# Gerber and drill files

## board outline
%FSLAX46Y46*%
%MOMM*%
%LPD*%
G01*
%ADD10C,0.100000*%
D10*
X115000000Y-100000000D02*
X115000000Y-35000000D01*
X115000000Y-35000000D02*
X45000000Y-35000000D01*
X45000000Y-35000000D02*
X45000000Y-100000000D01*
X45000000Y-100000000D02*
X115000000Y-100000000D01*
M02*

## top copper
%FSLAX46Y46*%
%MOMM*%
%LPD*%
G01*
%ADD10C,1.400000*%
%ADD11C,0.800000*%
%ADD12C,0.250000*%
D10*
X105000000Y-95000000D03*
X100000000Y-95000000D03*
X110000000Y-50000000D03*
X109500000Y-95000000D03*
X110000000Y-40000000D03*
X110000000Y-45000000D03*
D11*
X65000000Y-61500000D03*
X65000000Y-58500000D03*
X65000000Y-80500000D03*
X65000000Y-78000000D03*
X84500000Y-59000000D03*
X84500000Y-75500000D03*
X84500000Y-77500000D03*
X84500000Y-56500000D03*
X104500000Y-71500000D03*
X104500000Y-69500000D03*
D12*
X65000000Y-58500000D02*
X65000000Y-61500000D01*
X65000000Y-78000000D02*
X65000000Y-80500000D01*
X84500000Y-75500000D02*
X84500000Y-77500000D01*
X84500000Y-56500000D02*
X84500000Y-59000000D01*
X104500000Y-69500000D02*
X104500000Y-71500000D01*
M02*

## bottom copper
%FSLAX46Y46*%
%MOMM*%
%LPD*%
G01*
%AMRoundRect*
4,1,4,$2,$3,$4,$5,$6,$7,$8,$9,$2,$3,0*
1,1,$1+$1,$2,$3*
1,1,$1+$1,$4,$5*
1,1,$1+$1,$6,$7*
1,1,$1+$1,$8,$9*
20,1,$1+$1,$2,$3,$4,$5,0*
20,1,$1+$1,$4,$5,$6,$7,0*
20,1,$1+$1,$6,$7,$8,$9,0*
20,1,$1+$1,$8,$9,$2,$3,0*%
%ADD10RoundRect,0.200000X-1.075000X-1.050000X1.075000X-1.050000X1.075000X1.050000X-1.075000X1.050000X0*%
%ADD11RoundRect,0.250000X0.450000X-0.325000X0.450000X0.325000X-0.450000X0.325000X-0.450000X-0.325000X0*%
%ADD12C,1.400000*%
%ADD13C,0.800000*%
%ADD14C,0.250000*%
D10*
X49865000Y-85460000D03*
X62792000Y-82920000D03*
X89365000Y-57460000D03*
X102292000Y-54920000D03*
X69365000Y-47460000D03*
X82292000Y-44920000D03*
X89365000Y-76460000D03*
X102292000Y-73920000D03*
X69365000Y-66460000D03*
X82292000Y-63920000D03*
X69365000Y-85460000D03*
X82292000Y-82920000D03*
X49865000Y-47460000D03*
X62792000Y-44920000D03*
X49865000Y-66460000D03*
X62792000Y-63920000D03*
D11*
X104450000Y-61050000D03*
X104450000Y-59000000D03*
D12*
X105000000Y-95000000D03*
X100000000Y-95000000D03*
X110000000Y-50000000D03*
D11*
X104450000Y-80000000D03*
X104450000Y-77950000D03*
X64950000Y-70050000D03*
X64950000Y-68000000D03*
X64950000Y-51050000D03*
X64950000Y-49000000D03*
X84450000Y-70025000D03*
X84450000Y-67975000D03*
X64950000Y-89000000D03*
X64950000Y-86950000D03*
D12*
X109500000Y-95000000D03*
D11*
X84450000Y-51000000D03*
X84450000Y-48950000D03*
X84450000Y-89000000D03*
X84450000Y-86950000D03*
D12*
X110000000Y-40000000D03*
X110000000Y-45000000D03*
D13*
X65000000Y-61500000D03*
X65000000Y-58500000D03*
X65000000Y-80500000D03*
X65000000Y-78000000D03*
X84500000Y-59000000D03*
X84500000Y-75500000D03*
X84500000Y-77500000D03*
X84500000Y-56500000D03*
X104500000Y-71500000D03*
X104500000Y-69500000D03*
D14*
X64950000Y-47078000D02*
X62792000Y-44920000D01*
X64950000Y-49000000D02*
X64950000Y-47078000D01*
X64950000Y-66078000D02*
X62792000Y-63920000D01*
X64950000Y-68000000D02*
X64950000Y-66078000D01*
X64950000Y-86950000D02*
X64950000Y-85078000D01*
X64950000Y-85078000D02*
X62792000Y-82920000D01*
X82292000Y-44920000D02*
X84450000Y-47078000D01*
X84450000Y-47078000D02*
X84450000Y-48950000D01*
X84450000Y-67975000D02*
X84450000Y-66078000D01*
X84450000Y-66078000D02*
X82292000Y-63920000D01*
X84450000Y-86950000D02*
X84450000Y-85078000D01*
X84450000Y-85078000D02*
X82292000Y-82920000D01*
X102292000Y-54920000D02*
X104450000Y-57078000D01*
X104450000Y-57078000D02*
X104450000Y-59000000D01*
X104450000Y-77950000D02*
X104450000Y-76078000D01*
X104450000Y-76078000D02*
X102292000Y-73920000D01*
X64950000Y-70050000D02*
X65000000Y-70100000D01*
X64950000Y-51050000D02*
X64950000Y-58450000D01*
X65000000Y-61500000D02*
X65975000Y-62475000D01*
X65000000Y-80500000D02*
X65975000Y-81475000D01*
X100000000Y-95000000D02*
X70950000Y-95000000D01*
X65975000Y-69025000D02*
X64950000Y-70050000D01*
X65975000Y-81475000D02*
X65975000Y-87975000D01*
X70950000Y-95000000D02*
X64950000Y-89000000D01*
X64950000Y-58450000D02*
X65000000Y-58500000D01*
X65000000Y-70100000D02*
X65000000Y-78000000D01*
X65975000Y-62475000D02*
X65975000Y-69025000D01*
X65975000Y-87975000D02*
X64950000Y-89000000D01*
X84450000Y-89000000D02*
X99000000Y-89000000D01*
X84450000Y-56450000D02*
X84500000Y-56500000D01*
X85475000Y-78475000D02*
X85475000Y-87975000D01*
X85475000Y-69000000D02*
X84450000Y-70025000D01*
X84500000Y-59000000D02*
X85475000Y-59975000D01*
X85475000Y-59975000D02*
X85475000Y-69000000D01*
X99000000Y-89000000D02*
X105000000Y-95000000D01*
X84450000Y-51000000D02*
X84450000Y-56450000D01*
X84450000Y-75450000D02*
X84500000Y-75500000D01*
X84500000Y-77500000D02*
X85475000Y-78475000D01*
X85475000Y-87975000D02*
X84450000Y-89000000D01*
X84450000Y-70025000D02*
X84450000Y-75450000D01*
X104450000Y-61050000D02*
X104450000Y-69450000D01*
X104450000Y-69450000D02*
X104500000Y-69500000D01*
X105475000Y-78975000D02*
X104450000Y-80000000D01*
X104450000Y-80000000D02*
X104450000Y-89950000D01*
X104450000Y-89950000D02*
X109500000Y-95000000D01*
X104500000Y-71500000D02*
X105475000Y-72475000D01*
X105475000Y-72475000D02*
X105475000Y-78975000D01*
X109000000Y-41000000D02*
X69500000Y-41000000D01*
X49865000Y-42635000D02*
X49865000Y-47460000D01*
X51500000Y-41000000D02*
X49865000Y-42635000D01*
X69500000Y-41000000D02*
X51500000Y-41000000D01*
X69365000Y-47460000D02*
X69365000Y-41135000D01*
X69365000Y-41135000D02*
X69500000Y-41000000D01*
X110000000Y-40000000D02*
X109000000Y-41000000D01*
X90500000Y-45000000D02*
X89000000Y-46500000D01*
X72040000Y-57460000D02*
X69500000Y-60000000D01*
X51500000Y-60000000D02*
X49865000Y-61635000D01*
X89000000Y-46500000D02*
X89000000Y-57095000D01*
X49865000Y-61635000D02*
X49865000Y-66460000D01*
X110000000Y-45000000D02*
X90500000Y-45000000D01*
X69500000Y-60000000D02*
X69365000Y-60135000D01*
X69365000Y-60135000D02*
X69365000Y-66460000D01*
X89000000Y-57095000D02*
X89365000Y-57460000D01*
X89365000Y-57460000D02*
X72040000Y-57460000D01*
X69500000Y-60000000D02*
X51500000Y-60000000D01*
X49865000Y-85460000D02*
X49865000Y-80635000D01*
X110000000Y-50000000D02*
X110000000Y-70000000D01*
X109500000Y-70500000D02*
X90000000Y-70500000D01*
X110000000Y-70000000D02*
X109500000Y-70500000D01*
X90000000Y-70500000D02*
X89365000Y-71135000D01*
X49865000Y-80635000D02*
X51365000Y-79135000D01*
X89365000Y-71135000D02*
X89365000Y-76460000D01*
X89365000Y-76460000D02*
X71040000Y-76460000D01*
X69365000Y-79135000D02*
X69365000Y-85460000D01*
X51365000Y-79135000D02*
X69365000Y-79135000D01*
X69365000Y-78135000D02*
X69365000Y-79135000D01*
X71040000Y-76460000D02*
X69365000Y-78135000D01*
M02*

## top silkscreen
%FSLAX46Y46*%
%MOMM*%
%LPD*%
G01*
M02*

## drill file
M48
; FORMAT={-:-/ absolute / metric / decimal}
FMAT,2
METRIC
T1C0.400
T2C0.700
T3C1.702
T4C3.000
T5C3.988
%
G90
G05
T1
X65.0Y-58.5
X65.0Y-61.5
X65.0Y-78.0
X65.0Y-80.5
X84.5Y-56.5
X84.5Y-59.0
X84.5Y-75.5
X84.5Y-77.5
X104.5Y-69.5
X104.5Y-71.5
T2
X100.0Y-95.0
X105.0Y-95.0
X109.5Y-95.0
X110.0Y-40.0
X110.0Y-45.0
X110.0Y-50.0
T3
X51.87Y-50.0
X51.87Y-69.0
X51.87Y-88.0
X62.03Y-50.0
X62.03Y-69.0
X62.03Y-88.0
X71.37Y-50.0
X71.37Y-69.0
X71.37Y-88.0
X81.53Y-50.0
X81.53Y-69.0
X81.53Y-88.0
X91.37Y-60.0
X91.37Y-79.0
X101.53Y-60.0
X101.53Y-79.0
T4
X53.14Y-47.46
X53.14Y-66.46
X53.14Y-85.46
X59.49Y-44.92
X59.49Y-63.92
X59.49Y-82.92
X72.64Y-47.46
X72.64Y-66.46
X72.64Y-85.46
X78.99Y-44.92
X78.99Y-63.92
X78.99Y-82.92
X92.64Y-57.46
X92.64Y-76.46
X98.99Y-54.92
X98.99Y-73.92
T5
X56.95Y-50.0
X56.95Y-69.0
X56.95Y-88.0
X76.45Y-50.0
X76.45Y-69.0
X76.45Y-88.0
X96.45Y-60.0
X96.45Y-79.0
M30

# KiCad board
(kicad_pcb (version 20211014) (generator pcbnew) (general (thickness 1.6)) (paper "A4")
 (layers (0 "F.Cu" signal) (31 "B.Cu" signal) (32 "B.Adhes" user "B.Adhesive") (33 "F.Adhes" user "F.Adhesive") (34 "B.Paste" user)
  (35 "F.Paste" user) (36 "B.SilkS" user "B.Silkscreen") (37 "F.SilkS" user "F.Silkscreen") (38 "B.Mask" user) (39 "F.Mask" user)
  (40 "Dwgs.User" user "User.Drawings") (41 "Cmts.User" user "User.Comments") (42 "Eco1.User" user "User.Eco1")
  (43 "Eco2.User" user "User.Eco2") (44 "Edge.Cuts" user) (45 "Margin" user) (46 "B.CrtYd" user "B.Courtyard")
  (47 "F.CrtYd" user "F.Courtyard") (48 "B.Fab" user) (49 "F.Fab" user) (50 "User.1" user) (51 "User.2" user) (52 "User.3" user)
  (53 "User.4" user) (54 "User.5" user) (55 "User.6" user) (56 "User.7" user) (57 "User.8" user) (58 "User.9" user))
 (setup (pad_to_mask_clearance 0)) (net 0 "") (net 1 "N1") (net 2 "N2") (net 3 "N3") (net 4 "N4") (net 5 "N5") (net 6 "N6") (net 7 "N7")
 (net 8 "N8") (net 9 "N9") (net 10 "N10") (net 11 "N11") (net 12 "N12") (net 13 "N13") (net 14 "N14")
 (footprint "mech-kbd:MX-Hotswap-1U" (layer "F.Cu") (at 56.95 88)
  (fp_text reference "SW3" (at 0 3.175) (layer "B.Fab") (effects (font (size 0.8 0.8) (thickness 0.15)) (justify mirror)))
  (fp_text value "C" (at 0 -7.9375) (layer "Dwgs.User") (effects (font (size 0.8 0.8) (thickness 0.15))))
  (pad "" np_thru_hole circle (at 2.54 -5.08) (size 3 3) (drill 3) (layers F&B.Cu *.Mask))
  (pad "" np_thru_hole circle (at -3.81 -2.54) (size 3 3) (drill 3) (layers F&B.Cu *.Mask))
  (pad "" np_thru_hole circle (at 0 0) (size 3.9878 3.9878) (drill 3.9878) (layers F&B.Cu *.Mask))
  (pad "" np_thru_hole circle (at -5.08 0 48.099) (size 1.7018 1.7018) (drill 1.7018) (layers F&B.Cu *.Mask))
  (pad "" np_thru_hole circle (at 5.08 0 48.099) (size 1.7018 1.7018) (drill 1.7018) (layers F&B.Cu *.Mask))
  (pad "1" smd roundrect (at -7.085 -2.54) (size 2.55 2.5) (layers "B.Cu" "B.Paste" "B.Mask") (roundrect_rratio 0.08) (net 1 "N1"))
  (pad "2" smd roundrect (at 5.842 -5.08) (size 2.55 2.5) (layers "B.Cu" "B.Paste" "B.Mask") (roundrect_rratio 0.08) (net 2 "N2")))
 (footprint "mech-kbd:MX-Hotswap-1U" (layer "F.Cu") (at 96.45 60)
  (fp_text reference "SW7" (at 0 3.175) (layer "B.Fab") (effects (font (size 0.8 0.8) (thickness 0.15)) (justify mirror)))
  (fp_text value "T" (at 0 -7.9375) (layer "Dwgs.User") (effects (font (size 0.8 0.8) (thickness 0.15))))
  (pad "" np_thru_hole circle (at 5.08 0 48.099) (size 1.7018 1.7018) (drill 1.7018) (layers F&B.Cu *.Mask))
  (pad "" np_thru_hole circle (at 0 0) (size 3.9878 3.9878) (drill 3.9878) (layers F&B.Cu *.Mask))
  (pad "" np_thru_hole circle (at -3.81 -2.54) (size 3 3) (drill 3) (layers F&B.Cu *.Mask))
  (pad "" np_thru_hole circle (at 2.54 -5.08) (size 3 3) (drill 3) (layers F&B.Cu *.Mask))
  (pad "" np_thru_hole circle (at -5.08 0 48.099) (size 1.7018 1.7018) (drill 1.7018) (layers F&B.Cu *.Mask))
  (pad "1" smd roundrect (at -7.085 -2.54) (size 2.55 2.5) (layers "B.Cu" "B.Paste" "B.Mask") (roundrect_rratio 0.08) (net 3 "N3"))
  (pad "2" smd roundrect (at 5.842 -5.08) (size 2.55 2.5) (layers "B.Cu" "B.Paste" "B.Mask") (roundrect_rratio 0.08) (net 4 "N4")))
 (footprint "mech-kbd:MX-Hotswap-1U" (layer "F.Cu") (at 76.45 50)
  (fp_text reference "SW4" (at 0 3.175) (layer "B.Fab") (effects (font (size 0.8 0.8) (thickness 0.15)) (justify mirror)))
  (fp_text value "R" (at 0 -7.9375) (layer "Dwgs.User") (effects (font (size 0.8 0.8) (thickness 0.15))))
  (pad "" np_thru_hole circle (at 2.54 -5.08) (size 3 3) (drill 3) (layers F&B.Cu *.Mask))
  (pad "" np_thru_hole circle (at -3.81 -2.54) (size 3 3) (drill 3) (layers F&B.Cu *.Mask))
  (pad "" np_thru_hole circle (at 5.08 0 48.099) (size 1.7018 1.7018) (drill 1.7018) (layers F&B.Cu *.Mask))
  (pad "" np_thru_hole circle (at 0 0) (size 3.9878 3.9878) (drill 3.9878) (layers F&B.Cu *.Mask))
  (pad "" np_thru_hole circle (at -5.08 0 48.099) (size 1.7018 1.7018) (drill 1.7018) (layers F&B.Cu *.Mask))
  (pad "1" smd roundrect (at -7.085 -2.54) (size 2.55 2.5) (layers "B.Cu" "B.Paste" "B.Mask") (roundrect_rratio 0.08) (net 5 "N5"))
  (pad "2" smd roundrect (at 5.842 -5.08) (size 2.55 2.5) (layers "B.Cu" "B.Paste" "B.Mask") (roundrect_rratio 0.08) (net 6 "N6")))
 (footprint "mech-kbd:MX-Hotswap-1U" (layer "F.Cu") (at 96.45 79)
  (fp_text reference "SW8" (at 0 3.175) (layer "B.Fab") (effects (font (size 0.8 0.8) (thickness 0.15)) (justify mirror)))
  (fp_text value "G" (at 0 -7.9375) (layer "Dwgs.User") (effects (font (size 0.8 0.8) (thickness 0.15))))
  (pad "" np_thru_hole circle (at 0 0) (size 3.9878 3.9878) (drill 3.9878) (layers F&B.Cu *.Mask))
  (pad "" np_thru_hole circle (at 2.54 -5.08) (size 3 3) (drill 3) (layers F&B.Cu *.Mask))
  (pad "" np_thru_hole circle (at -3.81 -2.54) (size 3 3) (drill 3) (layers F&B.Cu *.Mask))
  (pad "" np_thru_hole circle (at 5.08 0 48.099) (size 1.7018 1.7018) (drill 1.7018) (layers F&B.Cu *.Mask))
  (pad "" np_thru_hole circle (at -5.08 0 48.099) (size 1.7018 1.7018) (drill 1.7018) (layers F&B.Cu *.Mask))
  (pad "1" smd roundrect (at -7.085 -2.54) (size 2.55 2.5) (layers "B.Cu" "B.Paste" "B.Mask") (roundrect_rratio 0.08) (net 1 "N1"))
  (pad "2" smd roundrect (at 5.842 -5.08) (size 2.55 2.5) (layers "B.Cu" "B.Paste" "B.Mask") (roundrect_rratio 0.08) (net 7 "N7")))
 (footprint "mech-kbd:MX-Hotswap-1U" (layer "F.Cu") (at 76.45 69)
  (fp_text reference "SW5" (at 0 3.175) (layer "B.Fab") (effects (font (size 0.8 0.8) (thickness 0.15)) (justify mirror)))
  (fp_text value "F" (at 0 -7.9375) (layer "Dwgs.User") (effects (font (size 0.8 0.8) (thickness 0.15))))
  (pad "" np_thru_hole circle (at 5.08 0 48.099) (size 1.7018 1.7018) (drill 1.7018) (layers F&B.Cu *.Mask))
  (pad "" np_thru_hole circle (at 2.54 -5.08) (size 3 3) (drill 3) (layers F&B.Cu *.Mask))
  (pad "" np_thru_hole circle (at -3.81 -2.54) (size 3 3) (drill 3) (layers F&B.Cu *.Mask))
  (pad "" np_thru_hole circle (at -5.08 0 48.099) (size 1.7018 1.7018) (drill 1.7018) (layers F&B.Cu *.Mask))
  (pad "" np_thru_hole circle (at 0 0) (size 3.9878 3.9878) (drill 3.9878) (layers F&B.Cu *.Mask))
  (pad "1" smd roundrect (at -7.085 -2.54) (size 2.55 2.5) (layers "B.Cu" "B.Paste" "B.Mask") (roundrect_rratio 0.08) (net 3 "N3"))
  (pad "2" smd roundrect (at 5.842 -5.08) (size 2.55 2.5) (layers "B.Cu" "B.Paste" "B.Mask") (roundrect_rratio 0.08) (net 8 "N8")))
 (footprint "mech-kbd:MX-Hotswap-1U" (layer "F.Cu") (at 76.45 88)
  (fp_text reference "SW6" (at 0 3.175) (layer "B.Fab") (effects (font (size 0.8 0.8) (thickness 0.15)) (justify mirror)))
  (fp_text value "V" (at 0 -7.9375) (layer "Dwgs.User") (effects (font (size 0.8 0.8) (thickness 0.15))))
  (pad "" np_thru_hole circle (at -3.81 -2.54) (size 3 3) (drill 3) (layers F&B.Cu *.Mask))
  (pad "" np_thru_hole circle (at 0 0) (size 3.9878 3.9878) (drill 3.9878) (layers F&B.Cu *.Mask))
  (pad "" np_thru_hole circle (at 5.08 0 48.099) (size 1.7018 1.7018) (drill 1.7018) (layers F&B.Cu *.Mask))
  (pad "" np_thru_hole circle (at -5.08 0 48.099) (size 1.7018 1.7018) (drill 1.7018) (layers F&B.Cu *.Mask))
  (pad "" np_thru_hole circle (at 2.54 -5.08) (size 3 3) (drill 3) (layers F&B.Cu *.Mask))
  (pad "1" smd roundrect (at -7.085 -2.54) (size 2.55 2.5) (layers "B.Cu" "B.Paste" "B.Mask") (roundrect_rratio 0.08) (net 1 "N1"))
  (pad "2" smd roundrect (at 5.842 -5.08) (size 2.55 2.5) (layers "B.Cu" "B.Paste" "B.Mask") (roundrect_rratio 0.08) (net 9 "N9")))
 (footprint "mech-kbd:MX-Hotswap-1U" (layer "F.Cu") (at 56.95 50)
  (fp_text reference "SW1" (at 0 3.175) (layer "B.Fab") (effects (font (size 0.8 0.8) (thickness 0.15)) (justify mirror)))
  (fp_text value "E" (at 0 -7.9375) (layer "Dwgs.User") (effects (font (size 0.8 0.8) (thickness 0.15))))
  (pad "" np_thru_hole circle (at 5.08 0 48.099) (size 1.7018 1.7018) (drill 1.7018) (layers F&B.Cu *.Mask))
  (pad "" np_thru_hole circle (at 2.54 -5.08) (size 3 3) (drill 3) (layers F&B.Cu *.Mask))
  (pad "" np_thru_hole circle (at -5.08 0 48.099) (size 1.7018 1.7018) (drill 1.7018) (layers F&B.Cu *.Mask))
  (pad "" np_thru_hole circle (at 0 0) (size 3.9878 3.9878) (drill 3.9878) (layers F&B.Cu *.Mask))
  (pad "" np_thru_hole circle (at -3.81 -2.54) (size 3 3) (drill 3) (layers F&B.Cu *.Mask))
  (pad "1" smd roundrect (at -7.085 -2.54) (size 2.55 2.5) (layers "B.Cu" "B.Paste" "B.Mask") (roundrect_rratio 0.08) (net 5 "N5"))
  (pad "2" smd roundrect (at 5.842 -5.08) (size 2.55 2.5) (layers "B.Cu" "B.Paste" "B.Mask") (roundrect_rratio 0.08) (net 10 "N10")))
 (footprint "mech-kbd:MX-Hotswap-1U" (layer "F.Cu") (at 56.95 69)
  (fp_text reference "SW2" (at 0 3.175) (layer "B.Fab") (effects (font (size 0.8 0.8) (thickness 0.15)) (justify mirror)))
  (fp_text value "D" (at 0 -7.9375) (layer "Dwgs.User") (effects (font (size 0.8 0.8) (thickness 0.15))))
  (pad "" np_thru_hole circle (at 0 0) (size 3.9878 3.9878) (drill 3.9878) (layers F&B.Cu *.Mask))
  (pad "" np_thru_hole circle (at -3.81 -2.54) (size 3 3) (drill 3) (layers F&B.Cu *.Mask))
  (pad "" np_thru_hole circle (at -5.08 0 48.099) (size 1.7018 1.7018) (drill 1.7018) (layers F&B.Cu *.Mask))
  (pad "" np_thru_hole circle (at 5.08 0 48.099) (size 1.7018 1.7018) (drill 1.7018) (layers F&B.Cu *.Mask))
  (pad "" np_thru_hole circle (at 2.54 -5.08) (size 3 3) (drill 3) (layers F&B.Cu *.Mask))
  (pad "1" smd roundrect (at -7.085 -2.54) (size 2.55 2.5) (layers "B.Cu" "B.Paste" "B.Mask") (roundrect_rratio 0.08) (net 3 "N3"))
  (pad "2" smd roundrect (at 5.842 -5.08) (size 2.55 2.5) (layers "B.Cu" "B.Paste" "B.Mask") (roundrect_rratio 0.08) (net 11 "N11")))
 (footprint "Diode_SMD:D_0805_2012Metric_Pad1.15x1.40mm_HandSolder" (layer "B.Cu") (at 104.45 60.025 90)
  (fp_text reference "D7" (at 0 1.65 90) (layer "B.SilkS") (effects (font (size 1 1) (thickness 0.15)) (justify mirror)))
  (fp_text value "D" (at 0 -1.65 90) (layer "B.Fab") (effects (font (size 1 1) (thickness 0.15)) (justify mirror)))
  (pad "1" smd roundrect (at -1.025 0 90) (size 1.15 1.4) (layers "B.Cu" "B.Paste" "B.Mask") (roundrect_rratio 0.2173913043) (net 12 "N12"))
  (pad "2" smd roundrect (at 1.025 0 90) (size 1.15 1.4) (layers "B.Cu" "B.Paste" "B.Mask") (roundrect_rratio 0.2173913043) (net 4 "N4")))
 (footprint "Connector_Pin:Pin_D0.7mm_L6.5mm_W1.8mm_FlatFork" (layer "B.Cu") (at 105 95 180)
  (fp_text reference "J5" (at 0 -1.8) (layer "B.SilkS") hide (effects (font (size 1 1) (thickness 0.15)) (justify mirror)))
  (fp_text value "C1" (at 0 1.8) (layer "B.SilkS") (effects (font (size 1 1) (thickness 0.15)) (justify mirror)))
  (pad "1" thru_hole circle (at 0 0 180) (size 1.4 1.4) (drill 0.7) (layers *.Cu *.Mask) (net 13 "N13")))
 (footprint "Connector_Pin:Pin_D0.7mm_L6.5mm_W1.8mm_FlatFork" (layer "B.Cu") (at 100 95 180)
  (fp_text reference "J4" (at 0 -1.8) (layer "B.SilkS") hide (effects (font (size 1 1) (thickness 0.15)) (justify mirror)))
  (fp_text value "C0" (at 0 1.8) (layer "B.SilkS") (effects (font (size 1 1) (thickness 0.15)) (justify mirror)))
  (pad "1" thru_hole circle (at 0 0 180) (size 1.4 1.4) (drill 0.7) (layers *.Cu *.Mask) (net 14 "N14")))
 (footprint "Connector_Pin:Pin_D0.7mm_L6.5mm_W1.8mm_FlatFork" (layer "B.Cu") (at 110 50 180)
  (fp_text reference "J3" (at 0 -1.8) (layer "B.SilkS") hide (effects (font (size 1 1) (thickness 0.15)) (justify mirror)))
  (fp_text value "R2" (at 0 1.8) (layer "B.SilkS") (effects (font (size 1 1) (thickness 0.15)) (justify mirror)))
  (pad "1" thru_hole circle (at 0 0 180) (size 1.4 1.4) (drill 0.7) (layers *.Cu *.Mask) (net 1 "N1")))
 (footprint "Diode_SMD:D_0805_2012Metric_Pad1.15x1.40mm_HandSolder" (layer "B.Cu") (at 104.45 78.975 90)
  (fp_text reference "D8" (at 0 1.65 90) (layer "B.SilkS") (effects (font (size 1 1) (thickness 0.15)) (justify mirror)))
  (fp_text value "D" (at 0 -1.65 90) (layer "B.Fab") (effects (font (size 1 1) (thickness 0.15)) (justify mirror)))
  (pad "1" smd roundrect (at -1.025 0 90) (size 1.15 1.4) (layers "B.Cu" "B.Paste" "B.Mask") (roundrect_rratio 0.2173913043) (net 12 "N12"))
  (pad "2" smd roundrect (at 1.025 0 90) (size 1.15 1.4) (layers "B.Cu" "B.Paste" "B.Mask") (roundrect_rratio 0.2173913043) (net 7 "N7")))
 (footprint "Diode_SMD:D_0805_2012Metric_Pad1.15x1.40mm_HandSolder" (layer "B.Cu") (at 64.95 69.025 90)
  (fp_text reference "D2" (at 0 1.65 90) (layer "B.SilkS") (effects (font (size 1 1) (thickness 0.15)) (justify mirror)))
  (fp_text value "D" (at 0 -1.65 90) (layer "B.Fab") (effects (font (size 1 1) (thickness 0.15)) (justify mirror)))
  (pad "1" smd roundrect (at -1.025 0 90) (size 1.15 1.4) (layers "B.Cu" "B.Paste" "B.Mask") (roundrect_rratio 0.2173913043) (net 14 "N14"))
  (pad "2" smd roundrect (at 1.025 0 90) (size 1.15 1.4) (layers "B.Cu" "B.Paste" "B.Mask") (roundrect_rratio 0.2173913043) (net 11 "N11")))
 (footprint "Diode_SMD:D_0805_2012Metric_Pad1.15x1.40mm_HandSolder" (layer "B.Cu") (at 64.95 50.025 90)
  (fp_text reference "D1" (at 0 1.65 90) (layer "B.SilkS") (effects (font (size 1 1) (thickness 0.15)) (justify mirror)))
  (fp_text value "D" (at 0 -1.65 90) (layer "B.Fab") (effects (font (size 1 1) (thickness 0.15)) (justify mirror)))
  (pad "1" smd roundrect (at -1.025 0 90) (size 1.15 1.4) (layers "B.Cu" "B.Paste" "B.Mask") (roundrect_rratio 0.2173913043) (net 14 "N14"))
  (pad "2" smd roundrect (at 1.025 0 90) (size 1.15 1.4) (layers "B.Cu" "B.Paste" "B.Mask") (roundrect_rratio 0.2173913043) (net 10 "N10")))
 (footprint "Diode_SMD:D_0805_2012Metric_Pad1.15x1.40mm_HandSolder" (layer "B.Cu") (at 84.45 69 90)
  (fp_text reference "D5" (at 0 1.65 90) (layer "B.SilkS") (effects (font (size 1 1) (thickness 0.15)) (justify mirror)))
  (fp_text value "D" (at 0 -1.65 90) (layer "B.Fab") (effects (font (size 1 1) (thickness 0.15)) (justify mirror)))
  (pad "1" smd roundrect (at -1.025 0 90) (size 1.15 1.4) (layers "B.Cu" "B.Paste" "B.Mask") (roundrect_rratio 0.2173913043) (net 13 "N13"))
  (pad "2" smd roundrect (at 1.025 0 90) (size 1.15 1.4) (layers "B.Cu" "B.Paste" "B.Mask") (roundrect_rratio 0.2173913043) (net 8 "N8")))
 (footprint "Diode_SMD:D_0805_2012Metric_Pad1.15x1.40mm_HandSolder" (layer "B.Cu") (at 64.95 87.975 90)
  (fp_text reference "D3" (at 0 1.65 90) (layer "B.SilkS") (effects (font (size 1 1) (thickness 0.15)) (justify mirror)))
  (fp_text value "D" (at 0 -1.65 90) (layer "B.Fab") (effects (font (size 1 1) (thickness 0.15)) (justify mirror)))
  (pad "1" smd roundrect (at -1.025 0 90) (size 1.15 1.4) (layers "B.Cu" "B.Paste" "B.Mask") (roundrect_rratio 0.2173913043) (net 14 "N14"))
  (pad "2" smd roundrect (at 1.025 0 90) (size 1.15 1.4) (layers "B.Cu" "B.Paste" "B.Mask") (roundrect_rratio 0.2173913043) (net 2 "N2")))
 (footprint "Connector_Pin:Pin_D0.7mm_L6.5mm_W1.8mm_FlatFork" (layer "B.Cu") (at 109.5 95 180)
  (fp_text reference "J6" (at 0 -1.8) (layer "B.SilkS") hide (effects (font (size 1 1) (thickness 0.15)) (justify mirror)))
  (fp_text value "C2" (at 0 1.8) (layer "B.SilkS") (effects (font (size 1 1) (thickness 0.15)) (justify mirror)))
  (pad "1" thru_hole circle (at 0 0 180) (size 1.4 1.4) (drill 0.7) (layers *.Cu *.Mask) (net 12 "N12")))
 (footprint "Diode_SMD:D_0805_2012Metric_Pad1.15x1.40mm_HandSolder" (layer "B.Cu") (at 84.45 49.975 90)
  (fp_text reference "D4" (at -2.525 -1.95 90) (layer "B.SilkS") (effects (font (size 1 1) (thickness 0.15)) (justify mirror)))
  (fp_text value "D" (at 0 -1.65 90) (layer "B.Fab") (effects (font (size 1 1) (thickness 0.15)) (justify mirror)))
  (pad "1" smd roundrect (at -1.025 0 90) (size 1.15 1.4) (layers "B.Cu" "B.Paste" "B.Mask") (roundrect_rratio 0.2173913043) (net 13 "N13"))
  (pad "2" smd roundrect (at 1.025 0 90) (size 1.15 1.4) (layers "B.Cu" "B.Paste" "B.Mask") (roundrect_rratio 0.2173913043) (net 6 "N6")))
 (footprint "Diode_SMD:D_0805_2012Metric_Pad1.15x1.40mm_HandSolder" (layer "B.Cu") (at 84.45 87.975 90)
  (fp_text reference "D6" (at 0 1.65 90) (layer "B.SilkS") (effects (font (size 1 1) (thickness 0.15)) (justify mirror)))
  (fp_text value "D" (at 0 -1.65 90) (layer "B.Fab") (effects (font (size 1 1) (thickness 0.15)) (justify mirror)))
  (pad "1" smd roundrect (at -1.025 0 90) (size 1.15 1.4) (layers "B.Cu" "B.Paste" "B.Mask") (roundrect_rratio 0.2173913043) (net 13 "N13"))
  (pad "2" smd roundrect (at 1.025 0 90) (size 1.15 1.4) (layers "B.Cu" "B.Paste" "B.Mask") (roundrect_rratio 0.2173913043) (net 9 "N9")))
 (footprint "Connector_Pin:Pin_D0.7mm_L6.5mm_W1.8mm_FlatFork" (layer "B.Cu") (at 110 40 180)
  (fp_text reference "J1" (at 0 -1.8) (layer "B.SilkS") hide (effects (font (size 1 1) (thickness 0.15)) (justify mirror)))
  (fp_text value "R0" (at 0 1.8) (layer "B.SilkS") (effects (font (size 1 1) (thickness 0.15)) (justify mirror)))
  (pad "1" thru_hole circle (at 0 0 180) (size 1.4 1.4) (drill 0.7) (layers *.Cu *.Mask) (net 5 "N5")))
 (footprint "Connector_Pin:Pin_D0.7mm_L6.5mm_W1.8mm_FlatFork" (layer "B.Cu") (at 110 45 180)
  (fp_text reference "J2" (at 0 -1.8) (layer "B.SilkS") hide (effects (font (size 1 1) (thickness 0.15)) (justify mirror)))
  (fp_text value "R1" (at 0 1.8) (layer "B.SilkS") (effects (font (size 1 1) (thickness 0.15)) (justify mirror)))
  (pad "1" thru_hole circle (at 0 0 180) (size 1.4 1.4) (drill 0.7) (layers *.Cu *.Mask) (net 3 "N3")))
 (gr_line (start 115 100) (end 115 35) (layer "Edge.Cuts") (width 0.1))
 (gr_line (start 115 35) (end 45 35) (layer "Edge.Cuts") (width 0.1))
 (gr_line (start 45 35) (end 45 100) (layer "Edge.Cuts") (width 0.1))
 (gr_line (start 45 100) (end 115 100) (layer "Edge.Cuts") (width 0.1))
 (segment (start 64.95 47.078) (end 62.792 44.92) (width 0.25) (layer "B.Cu") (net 10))
 (segment (start 64.95 49) (end 64.95 47.078) (width 0.25) (layer "B.Cu") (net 10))
 (segment (start 64.95 66.078) (end 62.792 63.92) (width 0.25) (layer "B.Cu") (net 11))
 (segment (start 64.95 68) (end 64.95 66.078) (width 0.25) (layer "B.Cu") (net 11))
 (segment (start 64.95 86.95) (end 64.95 85.078) (width 0.25) (layer "B.Cu") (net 2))
 (segment (start 64.95 85.078) (end 62.792 82.92) (width 0.25) (layer "B.Cu") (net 2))
 (segment (start 82.292 44.92) (end 84.45 47.078) (width 0.25) (layer "B.Cu") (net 6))
 (segment (start 84.45 47.078) (end 84.45 48.95) (width 0.25) (layer "B.Cu") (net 6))
 (segment (start 84.45 67.975) (end 84.45 66.078) (width 0.25) (layer "B.Cu") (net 8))
 (segment (start 84.45 66.078) (end 82.292 63.92) (width 0.25) (layer "B.Cu") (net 8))
 (segment (start 84.45 86.95) (end 84.45 85.078) (width 0.25) (layer "B.Cu") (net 9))
 (segment (start 84.45 85.078) (end 82.292 82.92) (width 0.25) (layer "B.Cu") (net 9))
 (segment (start 102.292 54.92) (end 104.45 57.078) (width 0.25) (layer "B.Cu") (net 4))
 (segment (start 104.45 57.078) (end 104.45 59) (width 0.25) (layer "B.Cu") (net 4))
 (segment (start 104.45 77.95) (end 104.45 76.078) (width 0.25) (layer "B.Cu") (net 7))
 (segment (start 104.45 76.078) (end 102.292 73.92) (width 0.25) (layer "B.Cu") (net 7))
 (segment (start 65 58.5) (end 65 61.5) (width 0.25) (layer "F.Cu") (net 14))
 (segment (start 65 78) (end 65 80.5) (width 0.25) (layer "F.Cu") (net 14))
 (via (at 65 61.5) (size 0.8) (drill 0.4) (layers "F.Cu" "B.Cu") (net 14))
 (via (at 65 58.5) (size 0.8) (drill 0.4) (layers "F.Cu" "B.Cu") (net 14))
 (via (at 65 80.5) (size 0.8) (drill 0.4) (layers "F.Cu" "B.Cu") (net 14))
 (via (at 65 78) (size 0.8) (drill 0.4) (layers "F.Cu" "B.Cu") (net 14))
 (segment (start 64.95 70.05) (end 65 70.1) (width 0.25) (layer "B.Cu") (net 14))
 (segment (start 64.95 51.05) (end 64.95 58.45) (width 0.25) (layer "B.Cu") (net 14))
 (segment (start 65 61.5) (end 65.975 62.475) (width 0.25) (layer "B.Cu") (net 14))
 (segment (start 65 80.5) (end 65.975 81.475) (width 0.25) (layer "B.Cu") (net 14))
 (segment (start 100 95) (end 70.95 95) (width 0.25) (layer "B.Cu") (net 14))
 (segment (start 65.975 69.025) (end 64.95 70.05) (width 0.25) (layer "B.Cu") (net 14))
 (segment (start 65.975 81.475) (end 65.975 87.975) (width 0.25) (layer "B.Cu") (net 14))
 (segment (start 70.95 95) (end 64.95 89) (width 0.25) (layer "B.Cu") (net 14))
 (segment (start 64.95 58.45) (end 65 58.5) (width 0.25) (layer "B.Cu") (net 14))
 (segment (start 65 70.1) (end 65 78) (width 0.25) (layer "B.Cu") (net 14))
 (segment (start 65.975 62.475) (end 65.975 69.025) (width 0.25) (layer "B.Cu") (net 14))
 (segment (start 65.975 87.975) (end 64.95 89) (width 0.25) (layer "B.Cu") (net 14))
 (segment (start 84.5 75.5) (end 84.5 77.5) (width 0.25) (layer "F.Cu") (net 13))
 (segment (start 84.5 56.5) (end 84.5 59) (width 0.25) (layer "F.Cu") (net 13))
 (via (at 84.5 59) (size 0.8) (drill 0.4) (layers "F.Cu" "B.Cu") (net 13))
 (via (at 84.5 75.5) (size 0.8) (drill 0.4) (layers "F.Cu" "B.Cu") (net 13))
 (via (at 84.5 77.5) (size 0.8) (drill 0.4) (layers "F.Cu" "B.Cu") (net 13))
 (via (at 84.5 56.5) (size 0.8) (drill 0.4) (layers "F.Cu" "B.Cu") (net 13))
 (segment (start 84.45 89) (end 99 89) (width 0.25) (layer "B.Cu") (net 13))
 (segment (start 84.45 56.45) (end 84.5 56.5) (width 0.25) (layer "B.Cu") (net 13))
 (segment (start 85.475 78.475) (end 85.475 87.975) (width 0.25) (layer "B.Cu") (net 13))
 (segment (start 85.475 69) (end 84.45 70.025) (width 0.25) (layer "B.Cu") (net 13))
 (segment (start 84.5 59) (end 85.475 59.975) (width 0.25) (layer "B.Cu") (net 13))
 (segment (start 85.475 59.975) (end 85.475 69) (width 0.25) (layer "B.Cu") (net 13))
 (segment (start 99 89) (end 105 95) (width 0.25) (layer "B.Cu") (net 13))
 (segment (start 84.45 51) (end 84.45 56.45) (width 0.25) (layer "B.Cu") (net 13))
 (segment (start 84.45 75.45) (end 84.5 75.5) (width 0.25) (layer "B.Cu") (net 13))
 (segment (start 84.5 77.5) (end 85.475 78.475) (width 0.25) (layer "B.Cu") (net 13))
 (segment (start 85.475 87.975) (end 84.45 89) (width 0.25) (layer "B.Cu") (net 13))
 (segment (start 84.45 70.025) (end 84.45 75.45) (width 0.25) (layer "B.Cu") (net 13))
 (segment (start 104.5 69.5) (end 104.5 71.5) (width 0.25) (layer "F.Cu") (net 12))
 (via (at 104.5 71.5) (size 0.8) (drill 0.4) (layers "F.Cu" "B.Cu") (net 12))
 (via (at 104.5 69.5) (size 0.8) (drill 0.4) (layers "F.Cu" "B.Cu") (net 12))
 (segment (start 104.45 61.05) (end 104.45 69.45) (width 0.25) (layer "B.Cu") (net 12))
 (segment (start 104.45 69.45) (end 104.5 69.5) (width 0.25) (layer "B.Cu") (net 12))
 (segment (start 105.475 78.975) (end 104.45 80) (width 0.25) (layer "B.Cu") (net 12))
 (segment (start 104.45 80) (end 104.45 89.95) (width 0.25) (layer "B.Cu") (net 12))
 (segment (start 104.45 89.95) (end 109.5 95) (width 0.25) (layer "B.Cu") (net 12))
 (segment (start 104.5 71.5) (end 105.475 72.475) (width 0.25) (layer "B.Cu") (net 12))
 (segment (start 105.475 72.475) (end 105.475 78.975) (width 0.25) (layer "B.Cu") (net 12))
 (segment (start 109 41) (end 69.5 41) (width 0.25) (layer "B.Cu") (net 5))
 (segment (start 49.865 42.635) (end 49.865 47.46) (width 0.25) (layer "B.Cu") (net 5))
 (segment (start 51.5 41) (end 49.865 42.635) (width 0.25) (layer "B.Cu") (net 5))
 (segment (start 69.5 41) (end 51.5 41) (width 0.25) (layer "B.Cu") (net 5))
 (segment (start 69.365 47.46) (end 69.365 41.135) (width 0.25) (layer "B.Cu") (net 5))
 (segment (start 69.365 41.135) (end 69.5 41) (width 0.25) (layer "B.Cu") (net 5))
 (segment (start 110 40) (end 109 41) (width 0.25) (layer "B.Cu") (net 5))
 (segment (start 90.5 45) (end 89 46.5) (width 0.25) (layer "B.Cu") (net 3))
 (segment (start 72.04 57.46) (end 69.5 60) (width 0.25) (layer "B.Cu") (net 3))
 (segment (start 51.5 60) (end 49.865 61.635) (width 0.25) (layer "B.Cu") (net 3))
 (segment (start 89 46.5) (end 89 57.095) (width 0.25) (layer "B.Cu") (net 3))
 (segment (start 49.865 61.635) (end 49.865 66.46) (width 0.25) (layer "B.Cu") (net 3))
 (segment (start 110 45) (end 90.5 45) (width 0.25) (layer "B.Cu") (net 3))
 (segment (start 69.5 60) (end 69.365 60.135) (width 0.25) (layer "B.Cu") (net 3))
 (segment (start 69.365 60.135) (end 69.365 66.46) (width 0.25) (layer "B.Cu") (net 3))
 (segment (start 89 57.095) (end 89.365 57.46) (width 0.25) (layer "B.Cu") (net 3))
 (segment (start 89.365 57.46) (end 72.04 57.46) (width 0.25) (layer "B.Cu") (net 3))
 (segment (start 69.5 60) (end 51.5 60) (width 0.25) (layer "B.Cu") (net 3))
 (segment (start 49.865 85.46) (end 49.865 80.635) (width 0.25) (layer "B.Cu") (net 1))
 (segment (start 110 50) (end 110 70) (width 0.25) (layer "B.Cu") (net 1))
 (segment (start 109.5 70.5) (end 90 70.5) (width 0.25) (layer "B.Cu") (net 1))
 (segment (start 110 70) (end 109.5 70.5) (width 0.25) (layer "B.Cu") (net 1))
 (segment (start 90 70.5) (end 89.365 71.135) (width 0.25) (layer "B.Cu") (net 1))
 (segment (start 49.865 80.635) (end 51.365 79.135) (width 0.25) (layer "B.Cu") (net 1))
 (segment (start 89.365 71.135) (end 89.365 76.46) (width 0.25) (layer "B.Cu") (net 1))
 (segment (start 89.365 76.46) (end 71.04 76.46) (width 0.25) (layer "B.Cu") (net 1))
 (segment (start 69.365 79.135) (end 69.365 85.46) (width 0.25) (layer "B.Cu") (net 1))
 (segment (start 51.365 79.135) (end 69.365 79.135) (width 0.25) (layer "B.Cu") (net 1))
 (segment (start 69.365 78.135) (end 69.365 79.135) (width 0.25) (layer "B.Cu") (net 1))
 (segment (start 71.04 76.46) (end 69.365 78.135) (width 0.25) (layer "B.Cu") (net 1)))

